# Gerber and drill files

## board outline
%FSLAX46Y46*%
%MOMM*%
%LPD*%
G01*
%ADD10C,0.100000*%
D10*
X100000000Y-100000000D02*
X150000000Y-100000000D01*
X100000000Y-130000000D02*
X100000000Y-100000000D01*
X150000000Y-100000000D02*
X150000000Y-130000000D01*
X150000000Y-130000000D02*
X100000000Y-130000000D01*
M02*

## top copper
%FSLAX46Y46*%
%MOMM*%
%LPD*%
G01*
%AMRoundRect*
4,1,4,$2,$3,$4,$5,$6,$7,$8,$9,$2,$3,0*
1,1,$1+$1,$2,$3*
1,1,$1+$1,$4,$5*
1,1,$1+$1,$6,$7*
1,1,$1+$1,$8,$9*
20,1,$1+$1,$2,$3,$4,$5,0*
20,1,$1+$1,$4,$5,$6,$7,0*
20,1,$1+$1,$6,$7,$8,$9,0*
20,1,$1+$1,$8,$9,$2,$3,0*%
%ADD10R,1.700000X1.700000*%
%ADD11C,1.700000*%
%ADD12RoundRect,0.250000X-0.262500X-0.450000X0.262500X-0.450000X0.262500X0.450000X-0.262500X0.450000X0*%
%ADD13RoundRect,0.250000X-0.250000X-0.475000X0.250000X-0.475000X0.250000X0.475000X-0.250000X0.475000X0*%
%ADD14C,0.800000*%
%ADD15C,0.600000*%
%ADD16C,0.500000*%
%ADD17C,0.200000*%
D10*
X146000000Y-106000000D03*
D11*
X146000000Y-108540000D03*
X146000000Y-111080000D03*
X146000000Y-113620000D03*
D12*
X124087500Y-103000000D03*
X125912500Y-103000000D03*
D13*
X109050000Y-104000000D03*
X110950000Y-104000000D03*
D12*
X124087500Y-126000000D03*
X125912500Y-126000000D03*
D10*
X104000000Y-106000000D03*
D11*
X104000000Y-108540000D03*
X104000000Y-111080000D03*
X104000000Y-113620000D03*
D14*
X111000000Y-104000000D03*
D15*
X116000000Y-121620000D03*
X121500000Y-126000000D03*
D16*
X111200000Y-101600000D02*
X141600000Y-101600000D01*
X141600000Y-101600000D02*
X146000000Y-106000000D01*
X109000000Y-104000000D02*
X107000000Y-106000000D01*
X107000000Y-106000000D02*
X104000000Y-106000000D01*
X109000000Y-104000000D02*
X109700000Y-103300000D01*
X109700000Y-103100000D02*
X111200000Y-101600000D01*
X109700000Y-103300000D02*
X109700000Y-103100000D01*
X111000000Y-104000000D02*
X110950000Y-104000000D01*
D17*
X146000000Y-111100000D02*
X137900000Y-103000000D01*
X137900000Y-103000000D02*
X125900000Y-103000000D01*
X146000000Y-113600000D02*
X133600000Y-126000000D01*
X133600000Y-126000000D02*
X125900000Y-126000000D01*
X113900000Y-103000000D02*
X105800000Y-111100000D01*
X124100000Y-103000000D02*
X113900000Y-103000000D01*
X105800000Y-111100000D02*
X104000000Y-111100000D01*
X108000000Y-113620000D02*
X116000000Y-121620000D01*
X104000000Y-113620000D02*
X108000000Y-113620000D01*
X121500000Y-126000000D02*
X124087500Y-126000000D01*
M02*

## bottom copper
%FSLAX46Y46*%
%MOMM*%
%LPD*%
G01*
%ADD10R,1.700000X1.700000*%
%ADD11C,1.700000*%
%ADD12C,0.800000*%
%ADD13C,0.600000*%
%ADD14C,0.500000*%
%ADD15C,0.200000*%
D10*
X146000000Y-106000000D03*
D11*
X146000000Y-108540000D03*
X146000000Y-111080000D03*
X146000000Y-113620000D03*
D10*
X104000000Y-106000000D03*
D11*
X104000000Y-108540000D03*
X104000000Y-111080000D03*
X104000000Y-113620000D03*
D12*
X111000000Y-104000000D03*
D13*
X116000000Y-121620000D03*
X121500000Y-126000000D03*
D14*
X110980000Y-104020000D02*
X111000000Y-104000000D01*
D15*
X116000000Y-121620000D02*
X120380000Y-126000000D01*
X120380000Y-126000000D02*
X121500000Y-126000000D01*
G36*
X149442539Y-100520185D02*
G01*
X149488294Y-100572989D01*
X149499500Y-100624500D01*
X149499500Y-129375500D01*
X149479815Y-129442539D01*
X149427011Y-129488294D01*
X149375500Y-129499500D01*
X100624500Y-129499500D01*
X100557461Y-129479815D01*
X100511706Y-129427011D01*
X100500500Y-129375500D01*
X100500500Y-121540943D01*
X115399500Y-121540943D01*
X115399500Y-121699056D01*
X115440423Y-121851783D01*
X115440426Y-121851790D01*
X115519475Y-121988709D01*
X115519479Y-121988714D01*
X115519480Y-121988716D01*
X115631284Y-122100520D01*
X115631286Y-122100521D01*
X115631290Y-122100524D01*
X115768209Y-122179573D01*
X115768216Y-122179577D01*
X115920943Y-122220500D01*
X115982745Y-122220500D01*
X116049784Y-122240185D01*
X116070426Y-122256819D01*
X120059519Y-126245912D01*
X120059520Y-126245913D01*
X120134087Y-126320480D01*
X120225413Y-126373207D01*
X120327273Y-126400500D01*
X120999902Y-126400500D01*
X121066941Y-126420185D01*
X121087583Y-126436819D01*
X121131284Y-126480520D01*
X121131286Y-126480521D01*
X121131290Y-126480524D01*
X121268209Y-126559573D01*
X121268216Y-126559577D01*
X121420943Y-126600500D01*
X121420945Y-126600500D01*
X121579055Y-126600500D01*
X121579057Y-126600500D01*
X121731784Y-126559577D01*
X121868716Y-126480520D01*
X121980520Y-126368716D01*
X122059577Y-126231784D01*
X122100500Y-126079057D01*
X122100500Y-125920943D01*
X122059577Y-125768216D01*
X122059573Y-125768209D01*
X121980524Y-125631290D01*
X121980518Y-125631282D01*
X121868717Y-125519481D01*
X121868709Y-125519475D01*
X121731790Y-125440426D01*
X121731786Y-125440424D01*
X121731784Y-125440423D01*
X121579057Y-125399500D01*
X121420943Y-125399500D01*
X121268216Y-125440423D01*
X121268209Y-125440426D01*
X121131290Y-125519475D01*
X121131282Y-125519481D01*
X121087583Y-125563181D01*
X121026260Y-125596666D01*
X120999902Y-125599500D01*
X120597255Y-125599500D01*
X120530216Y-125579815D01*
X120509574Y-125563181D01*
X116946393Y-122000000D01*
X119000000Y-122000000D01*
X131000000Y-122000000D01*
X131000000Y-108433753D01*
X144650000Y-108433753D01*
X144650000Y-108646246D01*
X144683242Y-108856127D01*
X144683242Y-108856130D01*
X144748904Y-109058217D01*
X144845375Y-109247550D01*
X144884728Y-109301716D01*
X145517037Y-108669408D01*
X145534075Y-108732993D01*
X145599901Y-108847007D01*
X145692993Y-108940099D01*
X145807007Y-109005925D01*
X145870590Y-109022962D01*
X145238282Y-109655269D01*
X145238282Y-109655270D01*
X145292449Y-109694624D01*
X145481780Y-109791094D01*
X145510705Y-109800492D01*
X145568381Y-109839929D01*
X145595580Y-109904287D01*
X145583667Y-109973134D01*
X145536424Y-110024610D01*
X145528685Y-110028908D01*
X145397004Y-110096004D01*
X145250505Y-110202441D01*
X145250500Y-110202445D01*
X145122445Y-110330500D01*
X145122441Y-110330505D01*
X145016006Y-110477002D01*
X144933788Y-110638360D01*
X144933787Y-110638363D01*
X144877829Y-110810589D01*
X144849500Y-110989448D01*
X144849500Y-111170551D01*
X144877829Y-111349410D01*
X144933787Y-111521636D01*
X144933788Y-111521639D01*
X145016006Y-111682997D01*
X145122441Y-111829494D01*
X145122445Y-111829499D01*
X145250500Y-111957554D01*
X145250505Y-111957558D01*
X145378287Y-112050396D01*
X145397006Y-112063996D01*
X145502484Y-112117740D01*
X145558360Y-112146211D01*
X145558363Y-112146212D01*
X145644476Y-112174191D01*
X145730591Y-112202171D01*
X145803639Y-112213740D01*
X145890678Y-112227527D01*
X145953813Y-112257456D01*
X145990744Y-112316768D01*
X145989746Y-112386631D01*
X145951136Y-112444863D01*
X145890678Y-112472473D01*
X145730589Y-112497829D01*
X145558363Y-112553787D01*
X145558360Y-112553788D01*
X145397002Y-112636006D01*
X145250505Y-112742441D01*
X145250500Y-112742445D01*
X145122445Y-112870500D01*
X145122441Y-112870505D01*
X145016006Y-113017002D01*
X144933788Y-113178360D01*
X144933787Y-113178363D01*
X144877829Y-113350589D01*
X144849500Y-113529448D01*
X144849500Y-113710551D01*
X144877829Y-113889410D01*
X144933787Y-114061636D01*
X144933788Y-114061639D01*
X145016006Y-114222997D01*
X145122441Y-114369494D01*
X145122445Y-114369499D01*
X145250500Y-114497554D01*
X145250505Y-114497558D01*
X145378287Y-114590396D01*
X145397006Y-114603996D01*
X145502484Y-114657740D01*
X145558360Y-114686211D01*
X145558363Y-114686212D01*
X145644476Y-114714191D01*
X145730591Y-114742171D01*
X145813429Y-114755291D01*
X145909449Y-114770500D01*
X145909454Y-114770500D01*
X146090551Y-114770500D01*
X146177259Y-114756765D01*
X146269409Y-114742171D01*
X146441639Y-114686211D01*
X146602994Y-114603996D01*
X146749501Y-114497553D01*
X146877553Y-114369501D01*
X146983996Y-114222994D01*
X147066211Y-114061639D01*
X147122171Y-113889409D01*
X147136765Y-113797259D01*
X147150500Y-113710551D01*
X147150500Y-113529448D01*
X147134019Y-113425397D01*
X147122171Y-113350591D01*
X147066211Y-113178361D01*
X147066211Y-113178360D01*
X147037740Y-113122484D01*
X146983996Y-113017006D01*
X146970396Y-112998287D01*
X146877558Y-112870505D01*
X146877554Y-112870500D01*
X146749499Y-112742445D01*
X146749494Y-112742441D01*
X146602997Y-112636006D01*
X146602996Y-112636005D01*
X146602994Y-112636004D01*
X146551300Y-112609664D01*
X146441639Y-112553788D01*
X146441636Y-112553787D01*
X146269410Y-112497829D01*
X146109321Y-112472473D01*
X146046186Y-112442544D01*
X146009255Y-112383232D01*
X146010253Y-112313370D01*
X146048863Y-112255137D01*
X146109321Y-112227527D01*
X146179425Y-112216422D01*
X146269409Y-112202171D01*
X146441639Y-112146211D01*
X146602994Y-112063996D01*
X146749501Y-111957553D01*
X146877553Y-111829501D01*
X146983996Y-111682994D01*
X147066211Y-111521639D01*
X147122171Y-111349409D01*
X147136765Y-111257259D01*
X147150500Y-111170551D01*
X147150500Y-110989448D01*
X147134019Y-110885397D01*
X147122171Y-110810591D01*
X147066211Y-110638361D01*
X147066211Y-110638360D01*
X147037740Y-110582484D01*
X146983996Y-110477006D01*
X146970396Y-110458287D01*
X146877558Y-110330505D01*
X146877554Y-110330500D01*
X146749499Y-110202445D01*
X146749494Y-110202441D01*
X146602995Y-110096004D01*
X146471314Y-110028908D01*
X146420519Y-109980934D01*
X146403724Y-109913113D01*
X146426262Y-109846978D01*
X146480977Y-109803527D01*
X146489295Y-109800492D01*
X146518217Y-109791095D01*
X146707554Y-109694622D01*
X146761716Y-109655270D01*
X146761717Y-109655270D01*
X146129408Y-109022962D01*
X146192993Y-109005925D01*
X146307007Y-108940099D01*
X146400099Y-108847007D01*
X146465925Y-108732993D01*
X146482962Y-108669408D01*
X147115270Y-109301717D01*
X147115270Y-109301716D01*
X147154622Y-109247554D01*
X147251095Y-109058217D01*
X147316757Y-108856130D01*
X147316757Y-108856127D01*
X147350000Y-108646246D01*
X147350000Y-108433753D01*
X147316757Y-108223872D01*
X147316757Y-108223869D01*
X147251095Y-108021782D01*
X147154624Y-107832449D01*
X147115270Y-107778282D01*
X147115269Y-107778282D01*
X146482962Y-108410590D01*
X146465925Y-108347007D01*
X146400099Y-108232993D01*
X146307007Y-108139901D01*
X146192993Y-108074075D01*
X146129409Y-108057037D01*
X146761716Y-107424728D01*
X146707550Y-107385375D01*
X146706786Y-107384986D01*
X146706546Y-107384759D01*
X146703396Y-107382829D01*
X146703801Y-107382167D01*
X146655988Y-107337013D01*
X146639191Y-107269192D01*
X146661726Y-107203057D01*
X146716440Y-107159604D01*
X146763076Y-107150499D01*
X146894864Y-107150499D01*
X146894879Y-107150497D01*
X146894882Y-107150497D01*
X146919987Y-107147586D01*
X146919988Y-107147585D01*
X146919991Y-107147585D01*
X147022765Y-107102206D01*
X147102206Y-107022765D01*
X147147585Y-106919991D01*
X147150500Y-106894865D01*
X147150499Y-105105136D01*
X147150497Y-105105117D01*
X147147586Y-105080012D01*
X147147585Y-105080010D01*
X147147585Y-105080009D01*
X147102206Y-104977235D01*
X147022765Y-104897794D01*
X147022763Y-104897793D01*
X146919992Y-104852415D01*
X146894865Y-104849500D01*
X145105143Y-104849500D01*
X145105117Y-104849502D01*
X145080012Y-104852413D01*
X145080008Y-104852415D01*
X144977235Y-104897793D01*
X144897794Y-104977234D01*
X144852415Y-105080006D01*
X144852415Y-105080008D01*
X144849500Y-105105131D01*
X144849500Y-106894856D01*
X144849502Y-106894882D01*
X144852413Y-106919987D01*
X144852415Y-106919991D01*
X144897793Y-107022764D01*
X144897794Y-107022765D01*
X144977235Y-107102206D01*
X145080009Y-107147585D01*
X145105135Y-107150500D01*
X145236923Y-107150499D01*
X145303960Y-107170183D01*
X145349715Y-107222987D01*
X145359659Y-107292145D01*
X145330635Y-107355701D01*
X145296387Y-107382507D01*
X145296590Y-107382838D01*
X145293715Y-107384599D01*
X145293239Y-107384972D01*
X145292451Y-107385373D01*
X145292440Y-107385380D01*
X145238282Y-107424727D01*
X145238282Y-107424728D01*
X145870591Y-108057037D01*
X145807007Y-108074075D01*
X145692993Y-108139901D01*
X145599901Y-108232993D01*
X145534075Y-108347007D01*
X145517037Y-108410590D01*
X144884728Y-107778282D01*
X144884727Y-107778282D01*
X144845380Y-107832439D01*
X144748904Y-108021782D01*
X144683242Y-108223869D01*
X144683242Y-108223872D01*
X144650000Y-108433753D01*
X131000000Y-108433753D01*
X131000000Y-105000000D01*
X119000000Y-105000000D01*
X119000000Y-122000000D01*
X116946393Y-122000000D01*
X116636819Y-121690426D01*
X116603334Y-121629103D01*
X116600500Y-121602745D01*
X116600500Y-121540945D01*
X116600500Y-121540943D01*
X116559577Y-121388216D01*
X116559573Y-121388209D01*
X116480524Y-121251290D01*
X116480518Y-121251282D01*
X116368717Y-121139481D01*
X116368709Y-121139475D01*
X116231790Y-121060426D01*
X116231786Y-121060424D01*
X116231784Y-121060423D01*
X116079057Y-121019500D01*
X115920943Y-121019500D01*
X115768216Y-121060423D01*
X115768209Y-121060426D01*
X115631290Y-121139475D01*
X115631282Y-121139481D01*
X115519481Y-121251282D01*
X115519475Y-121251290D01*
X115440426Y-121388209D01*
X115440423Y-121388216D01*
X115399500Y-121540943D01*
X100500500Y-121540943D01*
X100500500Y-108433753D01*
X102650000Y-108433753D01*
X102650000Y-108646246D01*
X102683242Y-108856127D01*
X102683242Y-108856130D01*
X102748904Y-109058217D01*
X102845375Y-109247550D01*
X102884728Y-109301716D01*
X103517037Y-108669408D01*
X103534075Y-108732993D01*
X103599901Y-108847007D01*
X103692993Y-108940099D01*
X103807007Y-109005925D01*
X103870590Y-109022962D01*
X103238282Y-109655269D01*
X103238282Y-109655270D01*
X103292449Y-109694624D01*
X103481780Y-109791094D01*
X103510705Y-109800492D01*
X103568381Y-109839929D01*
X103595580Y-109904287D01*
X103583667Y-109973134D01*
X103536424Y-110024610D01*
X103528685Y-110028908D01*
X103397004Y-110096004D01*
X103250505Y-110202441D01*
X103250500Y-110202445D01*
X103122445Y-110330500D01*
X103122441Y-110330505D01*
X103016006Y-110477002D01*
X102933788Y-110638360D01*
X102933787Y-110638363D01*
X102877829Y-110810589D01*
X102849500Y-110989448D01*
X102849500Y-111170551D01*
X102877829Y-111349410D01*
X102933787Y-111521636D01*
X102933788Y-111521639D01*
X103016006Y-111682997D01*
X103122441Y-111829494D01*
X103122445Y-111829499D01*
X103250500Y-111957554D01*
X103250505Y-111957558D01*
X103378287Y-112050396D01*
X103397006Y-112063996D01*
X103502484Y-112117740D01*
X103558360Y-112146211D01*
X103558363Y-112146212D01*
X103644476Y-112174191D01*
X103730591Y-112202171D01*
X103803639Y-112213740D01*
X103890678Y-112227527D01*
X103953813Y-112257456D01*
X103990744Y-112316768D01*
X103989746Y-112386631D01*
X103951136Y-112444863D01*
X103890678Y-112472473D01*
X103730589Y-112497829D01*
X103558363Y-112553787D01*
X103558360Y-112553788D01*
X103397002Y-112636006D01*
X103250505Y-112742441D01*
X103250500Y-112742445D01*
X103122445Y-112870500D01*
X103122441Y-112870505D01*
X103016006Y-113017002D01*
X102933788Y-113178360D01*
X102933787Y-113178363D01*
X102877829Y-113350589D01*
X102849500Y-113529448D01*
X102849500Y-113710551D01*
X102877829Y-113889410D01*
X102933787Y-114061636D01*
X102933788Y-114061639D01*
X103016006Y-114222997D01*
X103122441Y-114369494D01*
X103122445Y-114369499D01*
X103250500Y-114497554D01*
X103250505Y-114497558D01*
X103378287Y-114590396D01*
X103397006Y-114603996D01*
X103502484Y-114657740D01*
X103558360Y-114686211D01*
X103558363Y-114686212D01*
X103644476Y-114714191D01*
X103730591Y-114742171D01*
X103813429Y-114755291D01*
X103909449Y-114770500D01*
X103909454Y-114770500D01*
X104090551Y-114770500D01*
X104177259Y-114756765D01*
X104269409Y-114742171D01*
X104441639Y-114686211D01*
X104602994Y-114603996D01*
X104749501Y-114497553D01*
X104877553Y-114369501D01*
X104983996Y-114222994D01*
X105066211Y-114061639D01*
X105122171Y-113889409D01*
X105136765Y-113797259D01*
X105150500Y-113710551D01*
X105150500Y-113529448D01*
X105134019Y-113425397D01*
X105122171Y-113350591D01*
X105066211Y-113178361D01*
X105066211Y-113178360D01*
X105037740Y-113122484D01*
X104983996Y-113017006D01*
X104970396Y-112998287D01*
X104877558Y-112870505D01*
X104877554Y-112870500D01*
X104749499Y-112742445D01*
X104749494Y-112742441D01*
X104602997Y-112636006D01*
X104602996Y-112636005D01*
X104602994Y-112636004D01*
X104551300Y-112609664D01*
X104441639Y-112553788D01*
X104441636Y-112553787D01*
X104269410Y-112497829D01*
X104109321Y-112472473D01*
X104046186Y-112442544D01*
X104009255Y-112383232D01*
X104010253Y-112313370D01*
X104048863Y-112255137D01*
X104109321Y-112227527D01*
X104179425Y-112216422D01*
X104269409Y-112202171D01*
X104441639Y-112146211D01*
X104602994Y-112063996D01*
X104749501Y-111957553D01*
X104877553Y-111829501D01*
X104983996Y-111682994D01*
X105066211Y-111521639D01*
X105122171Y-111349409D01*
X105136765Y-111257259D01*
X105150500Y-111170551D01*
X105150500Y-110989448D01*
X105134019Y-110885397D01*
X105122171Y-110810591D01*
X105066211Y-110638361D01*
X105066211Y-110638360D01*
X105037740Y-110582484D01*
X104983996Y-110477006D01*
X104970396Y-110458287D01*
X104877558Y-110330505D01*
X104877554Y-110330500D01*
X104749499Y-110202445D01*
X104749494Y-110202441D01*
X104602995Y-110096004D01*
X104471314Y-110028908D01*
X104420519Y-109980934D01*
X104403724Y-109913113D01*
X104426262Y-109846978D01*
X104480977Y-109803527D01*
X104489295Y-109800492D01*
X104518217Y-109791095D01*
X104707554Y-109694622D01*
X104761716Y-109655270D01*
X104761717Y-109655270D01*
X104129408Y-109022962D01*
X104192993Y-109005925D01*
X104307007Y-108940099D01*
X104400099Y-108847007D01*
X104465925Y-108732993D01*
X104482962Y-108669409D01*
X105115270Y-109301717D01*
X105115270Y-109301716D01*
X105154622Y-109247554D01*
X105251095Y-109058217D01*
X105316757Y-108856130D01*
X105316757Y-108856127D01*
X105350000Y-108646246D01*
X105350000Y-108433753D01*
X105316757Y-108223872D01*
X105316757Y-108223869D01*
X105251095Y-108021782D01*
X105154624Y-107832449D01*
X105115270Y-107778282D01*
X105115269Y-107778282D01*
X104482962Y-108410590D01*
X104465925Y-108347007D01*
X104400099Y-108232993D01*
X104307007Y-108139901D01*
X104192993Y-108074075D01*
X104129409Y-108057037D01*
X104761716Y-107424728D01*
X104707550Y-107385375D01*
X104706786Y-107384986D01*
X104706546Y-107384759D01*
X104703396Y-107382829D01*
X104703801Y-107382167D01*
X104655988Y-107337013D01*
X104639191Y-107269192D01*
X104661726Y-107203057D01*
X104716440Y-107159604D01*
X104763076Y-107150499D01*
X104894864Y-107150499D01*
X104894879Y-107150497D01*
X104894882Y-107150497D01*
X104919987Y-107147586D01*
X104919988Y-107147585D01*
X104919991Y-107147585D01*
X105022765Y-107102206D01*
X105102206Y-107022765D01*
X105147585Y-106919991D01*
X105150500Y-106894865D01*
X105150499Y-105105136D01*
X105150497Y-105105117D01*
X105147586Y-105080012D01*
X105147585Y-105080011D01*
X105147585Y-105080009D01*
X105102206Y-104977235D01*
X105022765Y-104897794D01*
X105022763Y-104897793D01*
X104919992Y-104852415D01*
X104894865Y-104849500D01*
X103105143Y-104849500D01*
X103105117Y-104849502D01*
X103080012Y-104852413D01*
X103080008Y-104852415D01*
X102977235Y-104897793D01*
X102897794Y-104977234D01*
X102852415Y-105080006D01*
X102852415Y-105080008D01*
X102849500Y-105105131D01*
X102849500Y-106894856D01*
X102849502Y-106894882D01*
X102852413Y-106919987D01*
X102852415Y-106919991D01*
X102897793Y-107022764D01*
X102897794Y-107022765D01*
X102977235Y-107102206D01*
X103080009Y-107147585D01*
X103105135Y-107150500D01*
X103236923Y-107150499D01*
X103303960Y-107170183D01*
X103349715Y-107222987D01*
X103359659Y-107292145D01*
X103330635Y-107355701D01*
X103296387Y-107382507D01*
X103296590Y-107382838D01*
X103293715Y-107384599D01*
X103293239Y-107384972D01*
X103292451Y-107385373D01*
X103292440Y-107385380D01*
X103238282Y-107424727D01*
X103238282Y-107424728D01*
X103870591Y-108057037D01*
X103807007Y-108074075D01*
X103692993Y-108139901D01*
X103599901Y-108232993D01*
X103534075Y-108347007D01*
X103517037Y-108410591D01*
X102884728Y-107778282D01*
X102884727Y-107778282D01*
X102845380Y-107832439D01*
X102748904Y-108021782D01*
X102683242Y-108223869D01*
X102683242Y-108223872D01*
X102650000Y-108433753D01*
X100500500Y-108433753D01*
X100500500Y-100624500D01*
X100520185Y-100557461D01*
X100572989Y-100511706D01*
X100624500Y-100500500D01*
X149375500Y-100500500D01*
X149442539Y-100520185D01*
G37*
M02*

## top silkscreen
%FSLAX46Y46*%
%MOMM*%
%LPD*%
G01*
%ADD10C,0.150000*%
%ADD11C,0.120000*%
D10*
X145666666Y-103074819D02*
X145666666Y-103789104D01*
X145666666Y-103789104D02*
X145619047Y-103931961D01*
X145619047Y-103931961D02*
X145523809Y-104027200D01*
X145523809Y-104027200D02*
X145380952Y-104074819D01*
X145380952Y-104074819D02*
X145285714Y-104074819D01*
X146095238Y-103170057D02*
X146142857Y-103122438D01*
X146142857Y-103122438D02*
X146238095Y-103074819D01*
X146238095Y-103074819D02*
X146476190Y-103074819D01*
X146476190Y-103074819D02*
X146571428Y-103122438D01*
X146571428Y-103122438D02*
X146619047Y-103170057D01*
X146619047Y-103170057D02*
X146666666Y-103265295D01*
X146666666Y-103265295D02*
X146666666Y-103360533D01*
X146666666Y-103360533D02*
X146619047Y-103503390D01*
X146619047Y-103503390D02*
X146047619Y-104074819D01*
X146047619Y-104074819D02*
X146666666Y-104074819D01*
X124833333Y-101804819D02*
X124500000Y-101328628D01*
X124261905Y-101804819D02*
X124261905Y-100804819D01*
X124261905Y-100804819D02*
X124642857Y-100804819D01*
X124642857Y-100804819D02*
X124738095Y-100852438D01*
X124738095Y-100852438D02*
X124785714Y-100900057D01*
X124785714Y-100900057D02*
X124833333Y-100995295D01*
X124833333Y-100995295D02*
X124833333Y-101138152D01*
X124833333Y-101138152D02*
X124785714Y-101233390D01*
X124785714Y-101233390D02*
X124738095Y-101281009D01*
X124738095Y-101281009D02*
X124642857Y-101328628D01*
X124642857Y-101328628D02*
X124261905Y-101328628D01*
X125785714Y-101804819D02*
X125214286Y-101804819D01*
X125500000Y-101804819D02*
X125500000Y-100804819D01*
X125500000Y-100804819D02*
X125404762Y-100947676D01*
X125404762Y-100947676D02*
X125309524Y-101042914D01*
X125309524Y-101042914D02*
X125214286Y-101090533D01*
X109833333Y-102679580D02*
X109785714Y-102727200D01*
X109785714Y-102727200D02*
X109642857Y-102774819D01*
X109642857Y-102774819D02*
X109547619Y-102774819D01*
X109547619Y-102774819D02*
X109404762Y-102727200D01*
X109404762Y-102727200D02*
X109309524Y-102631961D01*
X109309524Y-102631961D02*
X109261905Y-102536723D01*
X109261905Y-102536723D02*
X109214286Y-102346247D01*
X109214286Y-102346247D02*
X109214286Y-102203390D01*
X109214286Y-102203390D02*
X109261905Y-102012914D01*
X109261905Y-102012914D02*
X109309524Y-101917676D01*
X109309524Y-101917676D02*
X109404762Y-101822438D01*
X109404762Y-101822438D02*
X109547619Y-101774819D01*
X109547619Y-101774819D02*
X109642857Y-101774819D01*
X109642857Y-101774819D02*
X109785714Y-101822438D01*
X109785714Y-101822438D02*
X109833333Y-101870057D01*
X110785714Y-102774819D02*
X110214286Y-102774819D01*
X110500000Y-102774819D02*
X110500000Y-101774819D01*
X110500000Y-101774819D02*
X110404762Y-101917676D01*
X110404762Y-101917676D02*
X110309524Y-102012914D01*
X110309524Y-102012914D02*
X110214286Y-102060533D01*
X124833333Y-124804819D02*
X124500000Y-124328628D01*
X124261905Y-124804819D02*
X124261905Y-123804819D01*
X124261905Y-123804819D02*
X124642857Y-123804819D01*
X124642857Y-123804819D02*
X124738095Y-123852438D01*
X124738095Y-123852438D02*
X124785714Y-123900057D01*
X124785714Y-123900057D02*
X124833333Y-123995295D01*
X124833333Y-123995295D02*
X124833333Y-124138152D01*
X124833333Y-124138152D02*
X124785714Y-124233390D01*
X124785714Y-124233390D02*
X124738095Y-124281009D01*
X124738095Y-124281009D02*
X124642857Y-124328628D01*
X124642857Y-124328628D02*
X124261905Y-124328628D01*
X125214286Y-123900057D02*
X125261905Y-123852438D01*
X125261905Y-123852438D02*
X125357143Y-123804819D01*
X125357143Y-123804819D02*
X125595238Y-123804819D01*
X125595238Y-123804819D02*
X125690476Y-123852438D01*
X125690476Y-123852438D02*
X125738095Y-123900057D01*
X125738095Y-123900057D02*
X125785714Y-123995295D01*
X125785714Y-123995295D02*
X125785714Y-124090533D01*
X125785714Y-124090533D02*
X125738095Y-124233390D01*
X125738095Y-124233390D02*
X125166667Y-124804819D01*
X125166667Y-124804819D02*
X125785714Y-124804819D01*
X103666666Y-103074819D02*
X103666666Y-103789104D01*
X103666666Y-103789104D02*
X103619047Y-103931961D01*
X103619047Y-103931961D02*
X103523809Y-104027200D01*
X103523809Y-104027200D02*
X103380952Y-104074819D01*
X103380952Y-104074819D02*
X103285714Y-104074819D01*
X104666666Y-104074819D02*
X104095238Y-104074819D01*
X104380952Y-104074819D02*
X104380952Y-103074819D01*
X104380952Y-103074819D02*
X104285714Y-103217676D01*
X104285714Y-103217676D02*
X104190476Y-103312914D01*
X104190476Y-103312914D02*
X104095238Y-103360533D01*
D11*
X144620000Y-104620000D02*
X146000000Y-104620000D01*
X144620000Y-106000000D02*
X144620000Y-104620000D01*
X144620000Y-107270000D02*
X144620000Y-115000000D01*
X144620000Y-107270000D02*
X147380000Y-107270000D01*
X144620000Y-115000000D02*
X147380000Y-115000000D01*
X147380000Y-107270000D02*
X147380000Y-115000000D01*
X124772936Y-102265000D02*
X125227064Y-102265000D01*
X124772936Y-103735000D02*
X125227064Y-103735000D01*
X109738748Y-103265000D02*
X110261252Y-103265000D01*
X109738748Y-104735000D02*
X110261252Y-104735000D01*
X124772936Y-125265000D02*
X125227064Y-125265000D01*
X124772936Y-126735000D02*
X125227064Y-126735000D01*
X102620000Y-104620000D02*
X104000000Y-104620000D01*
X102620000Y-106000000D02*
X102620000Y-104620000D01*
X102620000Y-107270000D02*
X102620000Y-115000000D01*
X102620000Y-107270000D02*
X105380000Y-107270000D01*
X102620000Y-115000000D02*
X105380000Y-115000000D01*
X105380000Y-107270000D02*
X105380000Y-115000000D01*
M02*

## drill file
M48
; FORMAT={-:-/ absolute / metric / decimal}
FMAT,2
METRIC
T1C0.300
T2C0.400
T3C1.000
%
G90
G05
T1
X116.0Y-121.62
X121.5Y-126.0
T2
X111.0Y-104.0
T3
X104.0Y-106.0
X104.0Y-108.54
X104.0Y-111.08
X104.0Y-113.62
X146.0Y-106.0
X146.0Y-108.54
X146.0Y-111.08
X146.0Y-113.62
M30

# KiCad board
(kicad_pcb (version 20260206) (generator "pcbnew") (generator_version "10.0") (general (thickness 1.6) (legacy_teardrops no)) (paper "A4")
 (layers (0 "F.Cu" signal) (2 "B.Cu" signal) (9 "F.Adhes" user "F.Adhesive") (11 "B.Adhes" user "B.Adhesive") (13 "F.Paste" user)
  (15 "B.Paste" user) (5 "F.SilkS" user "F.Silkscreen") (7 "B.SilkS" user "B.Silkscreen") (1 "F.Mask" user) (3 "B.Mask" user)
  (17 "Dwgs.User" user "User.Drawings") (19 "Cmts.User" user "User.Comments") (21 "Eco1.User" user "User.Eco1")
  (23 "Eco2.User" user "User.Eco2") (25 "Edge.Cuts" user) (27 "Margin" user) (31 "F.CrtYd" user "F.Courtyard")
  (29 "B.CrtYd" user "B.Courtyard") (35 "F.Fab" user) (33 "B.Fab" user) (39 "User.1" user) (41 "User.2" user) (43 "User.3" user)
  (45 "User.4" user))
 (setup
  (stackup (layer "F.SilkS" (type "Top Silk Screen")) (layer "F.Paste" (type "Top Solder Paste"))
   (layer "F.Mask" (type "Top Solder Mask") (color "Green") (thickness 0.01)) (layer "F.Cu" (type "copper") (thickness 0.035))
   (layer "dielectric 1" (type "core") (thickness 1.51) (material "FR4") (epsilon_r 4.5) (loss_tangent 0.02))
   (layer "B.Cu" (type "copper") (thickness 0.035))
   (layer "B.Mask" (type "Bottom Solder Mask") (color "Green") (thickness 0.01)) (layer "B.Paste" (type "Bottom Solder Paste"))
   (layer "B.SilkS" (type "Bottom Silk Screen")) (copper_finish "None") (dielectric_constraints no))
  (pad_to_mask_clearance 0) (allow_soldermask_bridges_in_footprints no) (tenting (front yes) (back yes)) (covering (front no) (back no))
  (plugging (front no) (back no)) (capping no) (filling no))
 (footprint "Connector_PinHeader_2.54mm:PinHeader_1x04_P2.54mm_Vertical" (layer "F.Cu") (at 146 106)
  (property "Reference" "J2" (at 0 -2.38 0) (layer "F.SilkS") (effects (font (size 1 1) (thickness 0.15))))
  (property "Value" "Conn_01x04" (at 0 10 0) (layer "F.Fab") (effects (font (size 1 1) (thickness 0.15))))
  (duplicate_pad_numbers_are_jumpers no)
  (fp_line (start -1.38 -1.38) (end 0 -1.38) (stroke (width 0.12) (type solid)) (layer "F.SilkS"))
  (fp_line (start -1.38 0) (end -1.38 -1.38) (stroke (width 0.12) (type solid)) (layer "F.SilkS"))
  (fp_line (start -1.38 1.27) (end -1.38 9) (stroke (width 0.12) (type solid)) (layer "F.SilkS"))
  (fp_line (start -1.38 1.27) (end 1.38 1.27) (stroke (width 0.12) (type solid)) (layer "F.SilkS"))
  (fp_line (start -1.38 9) (end 1.38 9) (stroke (width 0.12) (type solid)) (layer "F.SilkS"))
  (fp_line (start 1.38 1.27) (end 1.38 9) (stroke (width 0.12) (type solid)) (layer "F.SilkS"))
  (pad "1" thru_hole rect (at 0 0) (size 1.7 1.7) (drill 1) (layers "*.Cu" "*.Mask") (remove_unused_layers no) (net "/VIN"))
  (pad "2" thru_hole circle (at 0 2.54) (size 1.7 1.7) (drill 1) (layers "*.Cu" "*.Mask") (remove_unused_layers no) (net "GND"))
  (pad "3" thru_hole circle (at 0 5.08) (size 1.7 1.7) (drill 1) (layers "*.Cu" "*.Mask") (remove_unused_layers no) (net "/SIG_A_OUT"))
  (pad "4" thru_hole circle (at 0 7.62) (size 1.7 1.7) (drill 1) (layers "*.Cu" "*.Mask") (remove_unused_layers no) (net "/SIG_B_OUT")))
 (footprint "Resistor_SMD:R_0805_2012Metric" (layer "F.Cu") (at 125 103)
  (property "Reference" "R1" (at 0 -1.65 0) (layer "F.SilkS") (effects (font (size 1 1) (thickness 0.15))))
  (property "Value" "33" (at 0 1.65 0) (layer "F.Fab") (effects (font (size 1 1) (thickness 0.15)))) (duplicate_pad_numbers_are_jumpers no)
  (fp_line (start -0.227064 -0.735) (end 0.227064 -0.735) (stroke (width 0.12) (type solid)) (layer "F.SilkS"))
  (fp_line (start -0.227064 0.735) (end 0.227064 0.735) (stroke (width 0.12) (type solid)) (layer "F.SilkS"))
  (pad "1" smd roundrect (at -0.9125 0) (size 1.025 1.4) (layers "F.Cu" "F.Mask" "F.Paste") (roundrect_rratio 0.243902) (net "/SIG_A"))
  (pad "2" smd roundrect (at 0.9125 0) (size 1.025 1.4) (layers "F.Cu" "F.Mask" "F.Paste") (roundrect_rratio 0.243902) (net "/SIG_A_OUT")))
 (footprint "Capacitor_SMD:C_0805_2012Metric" (layer "F.Cu") (at 110 104)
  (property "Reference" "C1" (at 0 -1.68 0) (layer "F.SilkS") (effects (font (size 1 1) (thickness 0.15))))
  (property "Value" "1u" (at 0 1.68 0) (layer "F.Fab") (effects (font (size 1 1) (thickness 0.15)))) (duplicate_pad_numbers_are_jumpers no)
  (fp_line (start -0.261252 -0.735) (end 0.261252 -0.735) (stroke (width 0.12) (type solid)) (layer "F.SilkS"))
  (fp_line (start -0.261252 0.735) (end 0.261252 0.735) (stroke (width 0.12) (type solid)) (layer "F.SilkS"))
  (pad "1" smd roundrect (at -0.95 0) (size 1 1.45) (layers "F.Cu" "F.Mask" "F.Paste") (roundrect_rratio 0.25) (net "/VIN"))
  (pad "2" smd roundrect (at 0.95 0) (size 1 1.45) (layers "F.Cu" "F.Mask" "F.Paste") (roundrect_rratio 0.25) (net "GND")))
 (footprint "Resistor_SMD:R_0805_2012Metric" (layer "F.Cu") (at 125 126)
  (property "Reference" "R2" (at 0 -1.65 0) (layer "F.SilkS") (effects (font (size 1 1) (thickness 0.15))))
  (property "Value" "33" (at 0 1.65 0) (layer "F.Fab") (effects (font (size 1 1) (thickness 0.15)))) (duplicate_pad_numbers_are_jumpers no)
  (fp_line (start -0.227064 -0.735) (end 0.227064 -0.735) (stroke (width 0.12) (type solid)) (layer "F.SilkS"))
  (fp_line (start -0.227064 0.735) (end 0.227064 0.735) (stroke (width 0.12) (type solid)) (layer "F.SilkS"))
  (pad "1" smd roundrect (at -0.9125 0) (size 1.025 1.4) (layers "F.Cu" "F.Mask" "F.Paste") (roundrect_rratio 0.243902) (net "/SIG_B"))
  (pad "2" smd roundrect (at 0.9125 0) (size 1.025 1.4) (layers "F.Cu" "F.Mask" "F.Paste") (roundrect_rratio 0.243902) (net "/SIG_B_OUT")))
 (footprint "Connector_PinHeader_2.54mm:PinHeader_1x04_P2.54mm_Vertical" (layer "F.Cu") (at 104 106)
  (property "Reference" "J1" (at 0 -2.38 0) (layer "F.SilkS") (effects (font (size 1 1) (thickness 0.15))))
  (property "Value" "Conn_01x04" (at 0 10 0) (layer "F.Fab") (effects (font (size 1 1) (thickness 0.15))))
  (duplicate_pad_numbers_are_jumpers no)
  (fp_line (start -1.38 -1.38) (end 0 -1.38) (stroke (width 0.12) (type solid)) (layer "F.SilkS"))
  (fp_line (start -1.38 0) (end -1.38 -1.38) (stroke (width 0.12) (type solid)) (layer "F.SilkS"))
  (fp_line (start -1.38 1.27) (end -1.38 9) (stroke (width 0.12) (type solid)) (layer "F.SilkS"))
  (fp_line (start -1.38 1.27) (end 1.38 1.27) (stroke (width 0.12) (type solid)) (layer "F.SilkS"))
  (fp_line (start -1.38 9) (end 1.38 9) (stroke (width 0.12) (type solid)) (layer "F.SilkS"))
  (fp_line (start 1.38 1.27) (end 1.38 9) (stroke (width 0.12) (type solid)) (layer "F.SilkS"))
  (pad "1" thru_hole rect (at 0 0) (size 1.7 1.7) (drill 1) (layers "*.Cu" "*.Mask") (remove_unused_layers no) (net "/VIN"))
  (pad "2" thru_hole circle (at 0 2.54) (size 1.7 1.7) (drill 1) (layers "*.Cu" "*.Mask") (remove_unused_layers no) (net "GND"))
  (pad "3" thru_hole circle (at 0 5.08) (size 1.7 1.7) (drill 1) (layers "*.Cu" "*.Mask") (remove_unused_layers no) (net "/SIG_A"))
  (pad "4" thru_hole circle (at 0 7.62) (size 1.7 1.7) (drill 1) (layers "*.Cu" "*.Mask") (remove_unused_layers no) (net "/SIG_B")))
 (gr_line (start 100 100) (end 150 100) (stroke (width 0.1) (type default)) (layer "Edge.Cuts"))
 (gr_line (start 100 130) (end 100 100) (stroke (width 0.1) (type default)) (layer "Edge.Cuts"))
 (gr_line (start 150 100) (end 150 130) (stroke (width 0.1) (type default)) (layer "Edge.Cuts"))
 (gr_line (start 150 130) (end 100 130) (stroke (width 0.1) (type default)) (layer "Edge.Cuts"))
 (segment (start 111.2 101.6) (end 141.6 101.6) (width 0.5) (layer "F.Cu") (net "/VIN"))
 (segment (start 141.6 101.6) (end 146 106) (width 0.5) (layer "F.Cu") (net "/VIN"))
 (segment (start 109 104) (end 107 106) (width 0.5) (layer "F.Cu") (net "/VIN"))
 (segment (start 107 106) (end 104 106) (width 0.5) (layer "F.Cu") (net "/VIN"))
 (segment (start 109 104) (end 109.7 103.3) (width 0.5) (layer "F.Cu") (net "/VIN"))
 (segment (start 109.7 103.1) (end 111.2 101.6) (width 0.5) (layer "F.Cu") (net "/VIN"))
 (segment (start 109.7 103.3) (end 109.7 103.1) (width 0.5) (layer "F.Cu") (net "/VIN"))
 (segment (start 111 104) (end 110.95 104) (width 0.5) (layer "F.Cu") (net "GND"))
 (via (at 111 104) (size 0.8) (drill 0.4) (layers "F.Cu" "B.Cu") (capping yes) (filling yes) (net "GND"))
 (segment (start 110.98 104.02) (end 111 104) (width 0.5) (layer "B.Cu") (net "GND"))
 (segment (start 146 111.1) (end 137.9 103) (width 0.2) (layer "F.Cu") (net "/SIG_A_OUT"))
 (segment (start 137.9 103) (end 125.9 103) (width 0.2) (layer "F.Cu") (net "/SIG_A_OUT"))
 (segment (start 146 113.6) (end 133.6 126) (width 0.2) (layer "F.Cu") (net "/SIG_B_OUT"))
 (segment (start 133.6 126) (end 125.9 126) (width 0.2) (layer "F.Cu") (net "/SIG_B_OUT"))
 (segment (start 113.9 103) (end 105.8 111.1) (width 0.2) (layer "F.Cu") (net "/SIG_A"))
 (segment (start 124.1 103) (end 113.9 103) (width 0.2) (layer "F.Cu") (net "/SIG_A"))
 (segment (start 105.8 111.1) (end 104 111.1) (width 0.2) (layer "F.Cu") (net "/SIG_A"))
 (segment (start 108 113.62) (end 116 121.62) (width 0.2) (locked yes) (layer "F.Cu") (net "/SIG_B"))
 (segment (start 104 113.62) (end 108 113.62) (width 0.2) (locked yes) (layer "F.Cu") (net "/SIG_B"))
 (segment (start 121.5 126) (end 124.0875 126) (width 0.2) (locked yes) (layer "F.Cu") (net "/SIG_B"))
 (via (at 116 121.62) (size 0.6) (drill 0.3) (layers "F.Cu" "B.Cu") (locked yes) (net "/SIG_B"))
 (via (at 121.5 126) (size 0.6) (drill 0.3) (layers "F.Cu" "B.Cu") (locked yes) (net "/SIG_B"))
 (segment (start 116 121.62) (end 120.38 126) (width 0.2) (locked yes) (layer "B.Cu") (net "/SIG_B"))
 (segment (start 120.38 126) (end 121.5 126) (width 0.2) (locked yes) (layer "B.Cu") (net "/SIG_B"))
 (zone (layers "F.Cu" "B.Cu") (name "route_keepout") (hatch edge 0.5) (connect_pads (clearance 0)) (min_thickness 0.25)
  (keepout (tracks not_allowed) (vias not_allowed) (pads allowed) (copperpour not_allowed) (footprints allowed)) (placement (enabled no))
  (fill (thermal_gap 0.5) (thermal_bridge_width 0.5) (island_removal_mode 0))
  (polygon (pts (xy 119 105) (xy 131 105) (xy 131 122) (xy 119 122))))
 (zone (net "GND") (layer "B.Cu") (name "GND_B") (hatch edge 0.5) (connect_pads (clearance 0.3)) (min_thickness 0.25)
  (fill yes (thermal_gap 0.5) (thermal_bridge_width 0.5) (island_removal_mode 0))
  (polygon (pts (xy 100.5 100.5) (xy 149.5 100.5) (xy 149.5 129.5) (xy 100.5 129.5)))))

